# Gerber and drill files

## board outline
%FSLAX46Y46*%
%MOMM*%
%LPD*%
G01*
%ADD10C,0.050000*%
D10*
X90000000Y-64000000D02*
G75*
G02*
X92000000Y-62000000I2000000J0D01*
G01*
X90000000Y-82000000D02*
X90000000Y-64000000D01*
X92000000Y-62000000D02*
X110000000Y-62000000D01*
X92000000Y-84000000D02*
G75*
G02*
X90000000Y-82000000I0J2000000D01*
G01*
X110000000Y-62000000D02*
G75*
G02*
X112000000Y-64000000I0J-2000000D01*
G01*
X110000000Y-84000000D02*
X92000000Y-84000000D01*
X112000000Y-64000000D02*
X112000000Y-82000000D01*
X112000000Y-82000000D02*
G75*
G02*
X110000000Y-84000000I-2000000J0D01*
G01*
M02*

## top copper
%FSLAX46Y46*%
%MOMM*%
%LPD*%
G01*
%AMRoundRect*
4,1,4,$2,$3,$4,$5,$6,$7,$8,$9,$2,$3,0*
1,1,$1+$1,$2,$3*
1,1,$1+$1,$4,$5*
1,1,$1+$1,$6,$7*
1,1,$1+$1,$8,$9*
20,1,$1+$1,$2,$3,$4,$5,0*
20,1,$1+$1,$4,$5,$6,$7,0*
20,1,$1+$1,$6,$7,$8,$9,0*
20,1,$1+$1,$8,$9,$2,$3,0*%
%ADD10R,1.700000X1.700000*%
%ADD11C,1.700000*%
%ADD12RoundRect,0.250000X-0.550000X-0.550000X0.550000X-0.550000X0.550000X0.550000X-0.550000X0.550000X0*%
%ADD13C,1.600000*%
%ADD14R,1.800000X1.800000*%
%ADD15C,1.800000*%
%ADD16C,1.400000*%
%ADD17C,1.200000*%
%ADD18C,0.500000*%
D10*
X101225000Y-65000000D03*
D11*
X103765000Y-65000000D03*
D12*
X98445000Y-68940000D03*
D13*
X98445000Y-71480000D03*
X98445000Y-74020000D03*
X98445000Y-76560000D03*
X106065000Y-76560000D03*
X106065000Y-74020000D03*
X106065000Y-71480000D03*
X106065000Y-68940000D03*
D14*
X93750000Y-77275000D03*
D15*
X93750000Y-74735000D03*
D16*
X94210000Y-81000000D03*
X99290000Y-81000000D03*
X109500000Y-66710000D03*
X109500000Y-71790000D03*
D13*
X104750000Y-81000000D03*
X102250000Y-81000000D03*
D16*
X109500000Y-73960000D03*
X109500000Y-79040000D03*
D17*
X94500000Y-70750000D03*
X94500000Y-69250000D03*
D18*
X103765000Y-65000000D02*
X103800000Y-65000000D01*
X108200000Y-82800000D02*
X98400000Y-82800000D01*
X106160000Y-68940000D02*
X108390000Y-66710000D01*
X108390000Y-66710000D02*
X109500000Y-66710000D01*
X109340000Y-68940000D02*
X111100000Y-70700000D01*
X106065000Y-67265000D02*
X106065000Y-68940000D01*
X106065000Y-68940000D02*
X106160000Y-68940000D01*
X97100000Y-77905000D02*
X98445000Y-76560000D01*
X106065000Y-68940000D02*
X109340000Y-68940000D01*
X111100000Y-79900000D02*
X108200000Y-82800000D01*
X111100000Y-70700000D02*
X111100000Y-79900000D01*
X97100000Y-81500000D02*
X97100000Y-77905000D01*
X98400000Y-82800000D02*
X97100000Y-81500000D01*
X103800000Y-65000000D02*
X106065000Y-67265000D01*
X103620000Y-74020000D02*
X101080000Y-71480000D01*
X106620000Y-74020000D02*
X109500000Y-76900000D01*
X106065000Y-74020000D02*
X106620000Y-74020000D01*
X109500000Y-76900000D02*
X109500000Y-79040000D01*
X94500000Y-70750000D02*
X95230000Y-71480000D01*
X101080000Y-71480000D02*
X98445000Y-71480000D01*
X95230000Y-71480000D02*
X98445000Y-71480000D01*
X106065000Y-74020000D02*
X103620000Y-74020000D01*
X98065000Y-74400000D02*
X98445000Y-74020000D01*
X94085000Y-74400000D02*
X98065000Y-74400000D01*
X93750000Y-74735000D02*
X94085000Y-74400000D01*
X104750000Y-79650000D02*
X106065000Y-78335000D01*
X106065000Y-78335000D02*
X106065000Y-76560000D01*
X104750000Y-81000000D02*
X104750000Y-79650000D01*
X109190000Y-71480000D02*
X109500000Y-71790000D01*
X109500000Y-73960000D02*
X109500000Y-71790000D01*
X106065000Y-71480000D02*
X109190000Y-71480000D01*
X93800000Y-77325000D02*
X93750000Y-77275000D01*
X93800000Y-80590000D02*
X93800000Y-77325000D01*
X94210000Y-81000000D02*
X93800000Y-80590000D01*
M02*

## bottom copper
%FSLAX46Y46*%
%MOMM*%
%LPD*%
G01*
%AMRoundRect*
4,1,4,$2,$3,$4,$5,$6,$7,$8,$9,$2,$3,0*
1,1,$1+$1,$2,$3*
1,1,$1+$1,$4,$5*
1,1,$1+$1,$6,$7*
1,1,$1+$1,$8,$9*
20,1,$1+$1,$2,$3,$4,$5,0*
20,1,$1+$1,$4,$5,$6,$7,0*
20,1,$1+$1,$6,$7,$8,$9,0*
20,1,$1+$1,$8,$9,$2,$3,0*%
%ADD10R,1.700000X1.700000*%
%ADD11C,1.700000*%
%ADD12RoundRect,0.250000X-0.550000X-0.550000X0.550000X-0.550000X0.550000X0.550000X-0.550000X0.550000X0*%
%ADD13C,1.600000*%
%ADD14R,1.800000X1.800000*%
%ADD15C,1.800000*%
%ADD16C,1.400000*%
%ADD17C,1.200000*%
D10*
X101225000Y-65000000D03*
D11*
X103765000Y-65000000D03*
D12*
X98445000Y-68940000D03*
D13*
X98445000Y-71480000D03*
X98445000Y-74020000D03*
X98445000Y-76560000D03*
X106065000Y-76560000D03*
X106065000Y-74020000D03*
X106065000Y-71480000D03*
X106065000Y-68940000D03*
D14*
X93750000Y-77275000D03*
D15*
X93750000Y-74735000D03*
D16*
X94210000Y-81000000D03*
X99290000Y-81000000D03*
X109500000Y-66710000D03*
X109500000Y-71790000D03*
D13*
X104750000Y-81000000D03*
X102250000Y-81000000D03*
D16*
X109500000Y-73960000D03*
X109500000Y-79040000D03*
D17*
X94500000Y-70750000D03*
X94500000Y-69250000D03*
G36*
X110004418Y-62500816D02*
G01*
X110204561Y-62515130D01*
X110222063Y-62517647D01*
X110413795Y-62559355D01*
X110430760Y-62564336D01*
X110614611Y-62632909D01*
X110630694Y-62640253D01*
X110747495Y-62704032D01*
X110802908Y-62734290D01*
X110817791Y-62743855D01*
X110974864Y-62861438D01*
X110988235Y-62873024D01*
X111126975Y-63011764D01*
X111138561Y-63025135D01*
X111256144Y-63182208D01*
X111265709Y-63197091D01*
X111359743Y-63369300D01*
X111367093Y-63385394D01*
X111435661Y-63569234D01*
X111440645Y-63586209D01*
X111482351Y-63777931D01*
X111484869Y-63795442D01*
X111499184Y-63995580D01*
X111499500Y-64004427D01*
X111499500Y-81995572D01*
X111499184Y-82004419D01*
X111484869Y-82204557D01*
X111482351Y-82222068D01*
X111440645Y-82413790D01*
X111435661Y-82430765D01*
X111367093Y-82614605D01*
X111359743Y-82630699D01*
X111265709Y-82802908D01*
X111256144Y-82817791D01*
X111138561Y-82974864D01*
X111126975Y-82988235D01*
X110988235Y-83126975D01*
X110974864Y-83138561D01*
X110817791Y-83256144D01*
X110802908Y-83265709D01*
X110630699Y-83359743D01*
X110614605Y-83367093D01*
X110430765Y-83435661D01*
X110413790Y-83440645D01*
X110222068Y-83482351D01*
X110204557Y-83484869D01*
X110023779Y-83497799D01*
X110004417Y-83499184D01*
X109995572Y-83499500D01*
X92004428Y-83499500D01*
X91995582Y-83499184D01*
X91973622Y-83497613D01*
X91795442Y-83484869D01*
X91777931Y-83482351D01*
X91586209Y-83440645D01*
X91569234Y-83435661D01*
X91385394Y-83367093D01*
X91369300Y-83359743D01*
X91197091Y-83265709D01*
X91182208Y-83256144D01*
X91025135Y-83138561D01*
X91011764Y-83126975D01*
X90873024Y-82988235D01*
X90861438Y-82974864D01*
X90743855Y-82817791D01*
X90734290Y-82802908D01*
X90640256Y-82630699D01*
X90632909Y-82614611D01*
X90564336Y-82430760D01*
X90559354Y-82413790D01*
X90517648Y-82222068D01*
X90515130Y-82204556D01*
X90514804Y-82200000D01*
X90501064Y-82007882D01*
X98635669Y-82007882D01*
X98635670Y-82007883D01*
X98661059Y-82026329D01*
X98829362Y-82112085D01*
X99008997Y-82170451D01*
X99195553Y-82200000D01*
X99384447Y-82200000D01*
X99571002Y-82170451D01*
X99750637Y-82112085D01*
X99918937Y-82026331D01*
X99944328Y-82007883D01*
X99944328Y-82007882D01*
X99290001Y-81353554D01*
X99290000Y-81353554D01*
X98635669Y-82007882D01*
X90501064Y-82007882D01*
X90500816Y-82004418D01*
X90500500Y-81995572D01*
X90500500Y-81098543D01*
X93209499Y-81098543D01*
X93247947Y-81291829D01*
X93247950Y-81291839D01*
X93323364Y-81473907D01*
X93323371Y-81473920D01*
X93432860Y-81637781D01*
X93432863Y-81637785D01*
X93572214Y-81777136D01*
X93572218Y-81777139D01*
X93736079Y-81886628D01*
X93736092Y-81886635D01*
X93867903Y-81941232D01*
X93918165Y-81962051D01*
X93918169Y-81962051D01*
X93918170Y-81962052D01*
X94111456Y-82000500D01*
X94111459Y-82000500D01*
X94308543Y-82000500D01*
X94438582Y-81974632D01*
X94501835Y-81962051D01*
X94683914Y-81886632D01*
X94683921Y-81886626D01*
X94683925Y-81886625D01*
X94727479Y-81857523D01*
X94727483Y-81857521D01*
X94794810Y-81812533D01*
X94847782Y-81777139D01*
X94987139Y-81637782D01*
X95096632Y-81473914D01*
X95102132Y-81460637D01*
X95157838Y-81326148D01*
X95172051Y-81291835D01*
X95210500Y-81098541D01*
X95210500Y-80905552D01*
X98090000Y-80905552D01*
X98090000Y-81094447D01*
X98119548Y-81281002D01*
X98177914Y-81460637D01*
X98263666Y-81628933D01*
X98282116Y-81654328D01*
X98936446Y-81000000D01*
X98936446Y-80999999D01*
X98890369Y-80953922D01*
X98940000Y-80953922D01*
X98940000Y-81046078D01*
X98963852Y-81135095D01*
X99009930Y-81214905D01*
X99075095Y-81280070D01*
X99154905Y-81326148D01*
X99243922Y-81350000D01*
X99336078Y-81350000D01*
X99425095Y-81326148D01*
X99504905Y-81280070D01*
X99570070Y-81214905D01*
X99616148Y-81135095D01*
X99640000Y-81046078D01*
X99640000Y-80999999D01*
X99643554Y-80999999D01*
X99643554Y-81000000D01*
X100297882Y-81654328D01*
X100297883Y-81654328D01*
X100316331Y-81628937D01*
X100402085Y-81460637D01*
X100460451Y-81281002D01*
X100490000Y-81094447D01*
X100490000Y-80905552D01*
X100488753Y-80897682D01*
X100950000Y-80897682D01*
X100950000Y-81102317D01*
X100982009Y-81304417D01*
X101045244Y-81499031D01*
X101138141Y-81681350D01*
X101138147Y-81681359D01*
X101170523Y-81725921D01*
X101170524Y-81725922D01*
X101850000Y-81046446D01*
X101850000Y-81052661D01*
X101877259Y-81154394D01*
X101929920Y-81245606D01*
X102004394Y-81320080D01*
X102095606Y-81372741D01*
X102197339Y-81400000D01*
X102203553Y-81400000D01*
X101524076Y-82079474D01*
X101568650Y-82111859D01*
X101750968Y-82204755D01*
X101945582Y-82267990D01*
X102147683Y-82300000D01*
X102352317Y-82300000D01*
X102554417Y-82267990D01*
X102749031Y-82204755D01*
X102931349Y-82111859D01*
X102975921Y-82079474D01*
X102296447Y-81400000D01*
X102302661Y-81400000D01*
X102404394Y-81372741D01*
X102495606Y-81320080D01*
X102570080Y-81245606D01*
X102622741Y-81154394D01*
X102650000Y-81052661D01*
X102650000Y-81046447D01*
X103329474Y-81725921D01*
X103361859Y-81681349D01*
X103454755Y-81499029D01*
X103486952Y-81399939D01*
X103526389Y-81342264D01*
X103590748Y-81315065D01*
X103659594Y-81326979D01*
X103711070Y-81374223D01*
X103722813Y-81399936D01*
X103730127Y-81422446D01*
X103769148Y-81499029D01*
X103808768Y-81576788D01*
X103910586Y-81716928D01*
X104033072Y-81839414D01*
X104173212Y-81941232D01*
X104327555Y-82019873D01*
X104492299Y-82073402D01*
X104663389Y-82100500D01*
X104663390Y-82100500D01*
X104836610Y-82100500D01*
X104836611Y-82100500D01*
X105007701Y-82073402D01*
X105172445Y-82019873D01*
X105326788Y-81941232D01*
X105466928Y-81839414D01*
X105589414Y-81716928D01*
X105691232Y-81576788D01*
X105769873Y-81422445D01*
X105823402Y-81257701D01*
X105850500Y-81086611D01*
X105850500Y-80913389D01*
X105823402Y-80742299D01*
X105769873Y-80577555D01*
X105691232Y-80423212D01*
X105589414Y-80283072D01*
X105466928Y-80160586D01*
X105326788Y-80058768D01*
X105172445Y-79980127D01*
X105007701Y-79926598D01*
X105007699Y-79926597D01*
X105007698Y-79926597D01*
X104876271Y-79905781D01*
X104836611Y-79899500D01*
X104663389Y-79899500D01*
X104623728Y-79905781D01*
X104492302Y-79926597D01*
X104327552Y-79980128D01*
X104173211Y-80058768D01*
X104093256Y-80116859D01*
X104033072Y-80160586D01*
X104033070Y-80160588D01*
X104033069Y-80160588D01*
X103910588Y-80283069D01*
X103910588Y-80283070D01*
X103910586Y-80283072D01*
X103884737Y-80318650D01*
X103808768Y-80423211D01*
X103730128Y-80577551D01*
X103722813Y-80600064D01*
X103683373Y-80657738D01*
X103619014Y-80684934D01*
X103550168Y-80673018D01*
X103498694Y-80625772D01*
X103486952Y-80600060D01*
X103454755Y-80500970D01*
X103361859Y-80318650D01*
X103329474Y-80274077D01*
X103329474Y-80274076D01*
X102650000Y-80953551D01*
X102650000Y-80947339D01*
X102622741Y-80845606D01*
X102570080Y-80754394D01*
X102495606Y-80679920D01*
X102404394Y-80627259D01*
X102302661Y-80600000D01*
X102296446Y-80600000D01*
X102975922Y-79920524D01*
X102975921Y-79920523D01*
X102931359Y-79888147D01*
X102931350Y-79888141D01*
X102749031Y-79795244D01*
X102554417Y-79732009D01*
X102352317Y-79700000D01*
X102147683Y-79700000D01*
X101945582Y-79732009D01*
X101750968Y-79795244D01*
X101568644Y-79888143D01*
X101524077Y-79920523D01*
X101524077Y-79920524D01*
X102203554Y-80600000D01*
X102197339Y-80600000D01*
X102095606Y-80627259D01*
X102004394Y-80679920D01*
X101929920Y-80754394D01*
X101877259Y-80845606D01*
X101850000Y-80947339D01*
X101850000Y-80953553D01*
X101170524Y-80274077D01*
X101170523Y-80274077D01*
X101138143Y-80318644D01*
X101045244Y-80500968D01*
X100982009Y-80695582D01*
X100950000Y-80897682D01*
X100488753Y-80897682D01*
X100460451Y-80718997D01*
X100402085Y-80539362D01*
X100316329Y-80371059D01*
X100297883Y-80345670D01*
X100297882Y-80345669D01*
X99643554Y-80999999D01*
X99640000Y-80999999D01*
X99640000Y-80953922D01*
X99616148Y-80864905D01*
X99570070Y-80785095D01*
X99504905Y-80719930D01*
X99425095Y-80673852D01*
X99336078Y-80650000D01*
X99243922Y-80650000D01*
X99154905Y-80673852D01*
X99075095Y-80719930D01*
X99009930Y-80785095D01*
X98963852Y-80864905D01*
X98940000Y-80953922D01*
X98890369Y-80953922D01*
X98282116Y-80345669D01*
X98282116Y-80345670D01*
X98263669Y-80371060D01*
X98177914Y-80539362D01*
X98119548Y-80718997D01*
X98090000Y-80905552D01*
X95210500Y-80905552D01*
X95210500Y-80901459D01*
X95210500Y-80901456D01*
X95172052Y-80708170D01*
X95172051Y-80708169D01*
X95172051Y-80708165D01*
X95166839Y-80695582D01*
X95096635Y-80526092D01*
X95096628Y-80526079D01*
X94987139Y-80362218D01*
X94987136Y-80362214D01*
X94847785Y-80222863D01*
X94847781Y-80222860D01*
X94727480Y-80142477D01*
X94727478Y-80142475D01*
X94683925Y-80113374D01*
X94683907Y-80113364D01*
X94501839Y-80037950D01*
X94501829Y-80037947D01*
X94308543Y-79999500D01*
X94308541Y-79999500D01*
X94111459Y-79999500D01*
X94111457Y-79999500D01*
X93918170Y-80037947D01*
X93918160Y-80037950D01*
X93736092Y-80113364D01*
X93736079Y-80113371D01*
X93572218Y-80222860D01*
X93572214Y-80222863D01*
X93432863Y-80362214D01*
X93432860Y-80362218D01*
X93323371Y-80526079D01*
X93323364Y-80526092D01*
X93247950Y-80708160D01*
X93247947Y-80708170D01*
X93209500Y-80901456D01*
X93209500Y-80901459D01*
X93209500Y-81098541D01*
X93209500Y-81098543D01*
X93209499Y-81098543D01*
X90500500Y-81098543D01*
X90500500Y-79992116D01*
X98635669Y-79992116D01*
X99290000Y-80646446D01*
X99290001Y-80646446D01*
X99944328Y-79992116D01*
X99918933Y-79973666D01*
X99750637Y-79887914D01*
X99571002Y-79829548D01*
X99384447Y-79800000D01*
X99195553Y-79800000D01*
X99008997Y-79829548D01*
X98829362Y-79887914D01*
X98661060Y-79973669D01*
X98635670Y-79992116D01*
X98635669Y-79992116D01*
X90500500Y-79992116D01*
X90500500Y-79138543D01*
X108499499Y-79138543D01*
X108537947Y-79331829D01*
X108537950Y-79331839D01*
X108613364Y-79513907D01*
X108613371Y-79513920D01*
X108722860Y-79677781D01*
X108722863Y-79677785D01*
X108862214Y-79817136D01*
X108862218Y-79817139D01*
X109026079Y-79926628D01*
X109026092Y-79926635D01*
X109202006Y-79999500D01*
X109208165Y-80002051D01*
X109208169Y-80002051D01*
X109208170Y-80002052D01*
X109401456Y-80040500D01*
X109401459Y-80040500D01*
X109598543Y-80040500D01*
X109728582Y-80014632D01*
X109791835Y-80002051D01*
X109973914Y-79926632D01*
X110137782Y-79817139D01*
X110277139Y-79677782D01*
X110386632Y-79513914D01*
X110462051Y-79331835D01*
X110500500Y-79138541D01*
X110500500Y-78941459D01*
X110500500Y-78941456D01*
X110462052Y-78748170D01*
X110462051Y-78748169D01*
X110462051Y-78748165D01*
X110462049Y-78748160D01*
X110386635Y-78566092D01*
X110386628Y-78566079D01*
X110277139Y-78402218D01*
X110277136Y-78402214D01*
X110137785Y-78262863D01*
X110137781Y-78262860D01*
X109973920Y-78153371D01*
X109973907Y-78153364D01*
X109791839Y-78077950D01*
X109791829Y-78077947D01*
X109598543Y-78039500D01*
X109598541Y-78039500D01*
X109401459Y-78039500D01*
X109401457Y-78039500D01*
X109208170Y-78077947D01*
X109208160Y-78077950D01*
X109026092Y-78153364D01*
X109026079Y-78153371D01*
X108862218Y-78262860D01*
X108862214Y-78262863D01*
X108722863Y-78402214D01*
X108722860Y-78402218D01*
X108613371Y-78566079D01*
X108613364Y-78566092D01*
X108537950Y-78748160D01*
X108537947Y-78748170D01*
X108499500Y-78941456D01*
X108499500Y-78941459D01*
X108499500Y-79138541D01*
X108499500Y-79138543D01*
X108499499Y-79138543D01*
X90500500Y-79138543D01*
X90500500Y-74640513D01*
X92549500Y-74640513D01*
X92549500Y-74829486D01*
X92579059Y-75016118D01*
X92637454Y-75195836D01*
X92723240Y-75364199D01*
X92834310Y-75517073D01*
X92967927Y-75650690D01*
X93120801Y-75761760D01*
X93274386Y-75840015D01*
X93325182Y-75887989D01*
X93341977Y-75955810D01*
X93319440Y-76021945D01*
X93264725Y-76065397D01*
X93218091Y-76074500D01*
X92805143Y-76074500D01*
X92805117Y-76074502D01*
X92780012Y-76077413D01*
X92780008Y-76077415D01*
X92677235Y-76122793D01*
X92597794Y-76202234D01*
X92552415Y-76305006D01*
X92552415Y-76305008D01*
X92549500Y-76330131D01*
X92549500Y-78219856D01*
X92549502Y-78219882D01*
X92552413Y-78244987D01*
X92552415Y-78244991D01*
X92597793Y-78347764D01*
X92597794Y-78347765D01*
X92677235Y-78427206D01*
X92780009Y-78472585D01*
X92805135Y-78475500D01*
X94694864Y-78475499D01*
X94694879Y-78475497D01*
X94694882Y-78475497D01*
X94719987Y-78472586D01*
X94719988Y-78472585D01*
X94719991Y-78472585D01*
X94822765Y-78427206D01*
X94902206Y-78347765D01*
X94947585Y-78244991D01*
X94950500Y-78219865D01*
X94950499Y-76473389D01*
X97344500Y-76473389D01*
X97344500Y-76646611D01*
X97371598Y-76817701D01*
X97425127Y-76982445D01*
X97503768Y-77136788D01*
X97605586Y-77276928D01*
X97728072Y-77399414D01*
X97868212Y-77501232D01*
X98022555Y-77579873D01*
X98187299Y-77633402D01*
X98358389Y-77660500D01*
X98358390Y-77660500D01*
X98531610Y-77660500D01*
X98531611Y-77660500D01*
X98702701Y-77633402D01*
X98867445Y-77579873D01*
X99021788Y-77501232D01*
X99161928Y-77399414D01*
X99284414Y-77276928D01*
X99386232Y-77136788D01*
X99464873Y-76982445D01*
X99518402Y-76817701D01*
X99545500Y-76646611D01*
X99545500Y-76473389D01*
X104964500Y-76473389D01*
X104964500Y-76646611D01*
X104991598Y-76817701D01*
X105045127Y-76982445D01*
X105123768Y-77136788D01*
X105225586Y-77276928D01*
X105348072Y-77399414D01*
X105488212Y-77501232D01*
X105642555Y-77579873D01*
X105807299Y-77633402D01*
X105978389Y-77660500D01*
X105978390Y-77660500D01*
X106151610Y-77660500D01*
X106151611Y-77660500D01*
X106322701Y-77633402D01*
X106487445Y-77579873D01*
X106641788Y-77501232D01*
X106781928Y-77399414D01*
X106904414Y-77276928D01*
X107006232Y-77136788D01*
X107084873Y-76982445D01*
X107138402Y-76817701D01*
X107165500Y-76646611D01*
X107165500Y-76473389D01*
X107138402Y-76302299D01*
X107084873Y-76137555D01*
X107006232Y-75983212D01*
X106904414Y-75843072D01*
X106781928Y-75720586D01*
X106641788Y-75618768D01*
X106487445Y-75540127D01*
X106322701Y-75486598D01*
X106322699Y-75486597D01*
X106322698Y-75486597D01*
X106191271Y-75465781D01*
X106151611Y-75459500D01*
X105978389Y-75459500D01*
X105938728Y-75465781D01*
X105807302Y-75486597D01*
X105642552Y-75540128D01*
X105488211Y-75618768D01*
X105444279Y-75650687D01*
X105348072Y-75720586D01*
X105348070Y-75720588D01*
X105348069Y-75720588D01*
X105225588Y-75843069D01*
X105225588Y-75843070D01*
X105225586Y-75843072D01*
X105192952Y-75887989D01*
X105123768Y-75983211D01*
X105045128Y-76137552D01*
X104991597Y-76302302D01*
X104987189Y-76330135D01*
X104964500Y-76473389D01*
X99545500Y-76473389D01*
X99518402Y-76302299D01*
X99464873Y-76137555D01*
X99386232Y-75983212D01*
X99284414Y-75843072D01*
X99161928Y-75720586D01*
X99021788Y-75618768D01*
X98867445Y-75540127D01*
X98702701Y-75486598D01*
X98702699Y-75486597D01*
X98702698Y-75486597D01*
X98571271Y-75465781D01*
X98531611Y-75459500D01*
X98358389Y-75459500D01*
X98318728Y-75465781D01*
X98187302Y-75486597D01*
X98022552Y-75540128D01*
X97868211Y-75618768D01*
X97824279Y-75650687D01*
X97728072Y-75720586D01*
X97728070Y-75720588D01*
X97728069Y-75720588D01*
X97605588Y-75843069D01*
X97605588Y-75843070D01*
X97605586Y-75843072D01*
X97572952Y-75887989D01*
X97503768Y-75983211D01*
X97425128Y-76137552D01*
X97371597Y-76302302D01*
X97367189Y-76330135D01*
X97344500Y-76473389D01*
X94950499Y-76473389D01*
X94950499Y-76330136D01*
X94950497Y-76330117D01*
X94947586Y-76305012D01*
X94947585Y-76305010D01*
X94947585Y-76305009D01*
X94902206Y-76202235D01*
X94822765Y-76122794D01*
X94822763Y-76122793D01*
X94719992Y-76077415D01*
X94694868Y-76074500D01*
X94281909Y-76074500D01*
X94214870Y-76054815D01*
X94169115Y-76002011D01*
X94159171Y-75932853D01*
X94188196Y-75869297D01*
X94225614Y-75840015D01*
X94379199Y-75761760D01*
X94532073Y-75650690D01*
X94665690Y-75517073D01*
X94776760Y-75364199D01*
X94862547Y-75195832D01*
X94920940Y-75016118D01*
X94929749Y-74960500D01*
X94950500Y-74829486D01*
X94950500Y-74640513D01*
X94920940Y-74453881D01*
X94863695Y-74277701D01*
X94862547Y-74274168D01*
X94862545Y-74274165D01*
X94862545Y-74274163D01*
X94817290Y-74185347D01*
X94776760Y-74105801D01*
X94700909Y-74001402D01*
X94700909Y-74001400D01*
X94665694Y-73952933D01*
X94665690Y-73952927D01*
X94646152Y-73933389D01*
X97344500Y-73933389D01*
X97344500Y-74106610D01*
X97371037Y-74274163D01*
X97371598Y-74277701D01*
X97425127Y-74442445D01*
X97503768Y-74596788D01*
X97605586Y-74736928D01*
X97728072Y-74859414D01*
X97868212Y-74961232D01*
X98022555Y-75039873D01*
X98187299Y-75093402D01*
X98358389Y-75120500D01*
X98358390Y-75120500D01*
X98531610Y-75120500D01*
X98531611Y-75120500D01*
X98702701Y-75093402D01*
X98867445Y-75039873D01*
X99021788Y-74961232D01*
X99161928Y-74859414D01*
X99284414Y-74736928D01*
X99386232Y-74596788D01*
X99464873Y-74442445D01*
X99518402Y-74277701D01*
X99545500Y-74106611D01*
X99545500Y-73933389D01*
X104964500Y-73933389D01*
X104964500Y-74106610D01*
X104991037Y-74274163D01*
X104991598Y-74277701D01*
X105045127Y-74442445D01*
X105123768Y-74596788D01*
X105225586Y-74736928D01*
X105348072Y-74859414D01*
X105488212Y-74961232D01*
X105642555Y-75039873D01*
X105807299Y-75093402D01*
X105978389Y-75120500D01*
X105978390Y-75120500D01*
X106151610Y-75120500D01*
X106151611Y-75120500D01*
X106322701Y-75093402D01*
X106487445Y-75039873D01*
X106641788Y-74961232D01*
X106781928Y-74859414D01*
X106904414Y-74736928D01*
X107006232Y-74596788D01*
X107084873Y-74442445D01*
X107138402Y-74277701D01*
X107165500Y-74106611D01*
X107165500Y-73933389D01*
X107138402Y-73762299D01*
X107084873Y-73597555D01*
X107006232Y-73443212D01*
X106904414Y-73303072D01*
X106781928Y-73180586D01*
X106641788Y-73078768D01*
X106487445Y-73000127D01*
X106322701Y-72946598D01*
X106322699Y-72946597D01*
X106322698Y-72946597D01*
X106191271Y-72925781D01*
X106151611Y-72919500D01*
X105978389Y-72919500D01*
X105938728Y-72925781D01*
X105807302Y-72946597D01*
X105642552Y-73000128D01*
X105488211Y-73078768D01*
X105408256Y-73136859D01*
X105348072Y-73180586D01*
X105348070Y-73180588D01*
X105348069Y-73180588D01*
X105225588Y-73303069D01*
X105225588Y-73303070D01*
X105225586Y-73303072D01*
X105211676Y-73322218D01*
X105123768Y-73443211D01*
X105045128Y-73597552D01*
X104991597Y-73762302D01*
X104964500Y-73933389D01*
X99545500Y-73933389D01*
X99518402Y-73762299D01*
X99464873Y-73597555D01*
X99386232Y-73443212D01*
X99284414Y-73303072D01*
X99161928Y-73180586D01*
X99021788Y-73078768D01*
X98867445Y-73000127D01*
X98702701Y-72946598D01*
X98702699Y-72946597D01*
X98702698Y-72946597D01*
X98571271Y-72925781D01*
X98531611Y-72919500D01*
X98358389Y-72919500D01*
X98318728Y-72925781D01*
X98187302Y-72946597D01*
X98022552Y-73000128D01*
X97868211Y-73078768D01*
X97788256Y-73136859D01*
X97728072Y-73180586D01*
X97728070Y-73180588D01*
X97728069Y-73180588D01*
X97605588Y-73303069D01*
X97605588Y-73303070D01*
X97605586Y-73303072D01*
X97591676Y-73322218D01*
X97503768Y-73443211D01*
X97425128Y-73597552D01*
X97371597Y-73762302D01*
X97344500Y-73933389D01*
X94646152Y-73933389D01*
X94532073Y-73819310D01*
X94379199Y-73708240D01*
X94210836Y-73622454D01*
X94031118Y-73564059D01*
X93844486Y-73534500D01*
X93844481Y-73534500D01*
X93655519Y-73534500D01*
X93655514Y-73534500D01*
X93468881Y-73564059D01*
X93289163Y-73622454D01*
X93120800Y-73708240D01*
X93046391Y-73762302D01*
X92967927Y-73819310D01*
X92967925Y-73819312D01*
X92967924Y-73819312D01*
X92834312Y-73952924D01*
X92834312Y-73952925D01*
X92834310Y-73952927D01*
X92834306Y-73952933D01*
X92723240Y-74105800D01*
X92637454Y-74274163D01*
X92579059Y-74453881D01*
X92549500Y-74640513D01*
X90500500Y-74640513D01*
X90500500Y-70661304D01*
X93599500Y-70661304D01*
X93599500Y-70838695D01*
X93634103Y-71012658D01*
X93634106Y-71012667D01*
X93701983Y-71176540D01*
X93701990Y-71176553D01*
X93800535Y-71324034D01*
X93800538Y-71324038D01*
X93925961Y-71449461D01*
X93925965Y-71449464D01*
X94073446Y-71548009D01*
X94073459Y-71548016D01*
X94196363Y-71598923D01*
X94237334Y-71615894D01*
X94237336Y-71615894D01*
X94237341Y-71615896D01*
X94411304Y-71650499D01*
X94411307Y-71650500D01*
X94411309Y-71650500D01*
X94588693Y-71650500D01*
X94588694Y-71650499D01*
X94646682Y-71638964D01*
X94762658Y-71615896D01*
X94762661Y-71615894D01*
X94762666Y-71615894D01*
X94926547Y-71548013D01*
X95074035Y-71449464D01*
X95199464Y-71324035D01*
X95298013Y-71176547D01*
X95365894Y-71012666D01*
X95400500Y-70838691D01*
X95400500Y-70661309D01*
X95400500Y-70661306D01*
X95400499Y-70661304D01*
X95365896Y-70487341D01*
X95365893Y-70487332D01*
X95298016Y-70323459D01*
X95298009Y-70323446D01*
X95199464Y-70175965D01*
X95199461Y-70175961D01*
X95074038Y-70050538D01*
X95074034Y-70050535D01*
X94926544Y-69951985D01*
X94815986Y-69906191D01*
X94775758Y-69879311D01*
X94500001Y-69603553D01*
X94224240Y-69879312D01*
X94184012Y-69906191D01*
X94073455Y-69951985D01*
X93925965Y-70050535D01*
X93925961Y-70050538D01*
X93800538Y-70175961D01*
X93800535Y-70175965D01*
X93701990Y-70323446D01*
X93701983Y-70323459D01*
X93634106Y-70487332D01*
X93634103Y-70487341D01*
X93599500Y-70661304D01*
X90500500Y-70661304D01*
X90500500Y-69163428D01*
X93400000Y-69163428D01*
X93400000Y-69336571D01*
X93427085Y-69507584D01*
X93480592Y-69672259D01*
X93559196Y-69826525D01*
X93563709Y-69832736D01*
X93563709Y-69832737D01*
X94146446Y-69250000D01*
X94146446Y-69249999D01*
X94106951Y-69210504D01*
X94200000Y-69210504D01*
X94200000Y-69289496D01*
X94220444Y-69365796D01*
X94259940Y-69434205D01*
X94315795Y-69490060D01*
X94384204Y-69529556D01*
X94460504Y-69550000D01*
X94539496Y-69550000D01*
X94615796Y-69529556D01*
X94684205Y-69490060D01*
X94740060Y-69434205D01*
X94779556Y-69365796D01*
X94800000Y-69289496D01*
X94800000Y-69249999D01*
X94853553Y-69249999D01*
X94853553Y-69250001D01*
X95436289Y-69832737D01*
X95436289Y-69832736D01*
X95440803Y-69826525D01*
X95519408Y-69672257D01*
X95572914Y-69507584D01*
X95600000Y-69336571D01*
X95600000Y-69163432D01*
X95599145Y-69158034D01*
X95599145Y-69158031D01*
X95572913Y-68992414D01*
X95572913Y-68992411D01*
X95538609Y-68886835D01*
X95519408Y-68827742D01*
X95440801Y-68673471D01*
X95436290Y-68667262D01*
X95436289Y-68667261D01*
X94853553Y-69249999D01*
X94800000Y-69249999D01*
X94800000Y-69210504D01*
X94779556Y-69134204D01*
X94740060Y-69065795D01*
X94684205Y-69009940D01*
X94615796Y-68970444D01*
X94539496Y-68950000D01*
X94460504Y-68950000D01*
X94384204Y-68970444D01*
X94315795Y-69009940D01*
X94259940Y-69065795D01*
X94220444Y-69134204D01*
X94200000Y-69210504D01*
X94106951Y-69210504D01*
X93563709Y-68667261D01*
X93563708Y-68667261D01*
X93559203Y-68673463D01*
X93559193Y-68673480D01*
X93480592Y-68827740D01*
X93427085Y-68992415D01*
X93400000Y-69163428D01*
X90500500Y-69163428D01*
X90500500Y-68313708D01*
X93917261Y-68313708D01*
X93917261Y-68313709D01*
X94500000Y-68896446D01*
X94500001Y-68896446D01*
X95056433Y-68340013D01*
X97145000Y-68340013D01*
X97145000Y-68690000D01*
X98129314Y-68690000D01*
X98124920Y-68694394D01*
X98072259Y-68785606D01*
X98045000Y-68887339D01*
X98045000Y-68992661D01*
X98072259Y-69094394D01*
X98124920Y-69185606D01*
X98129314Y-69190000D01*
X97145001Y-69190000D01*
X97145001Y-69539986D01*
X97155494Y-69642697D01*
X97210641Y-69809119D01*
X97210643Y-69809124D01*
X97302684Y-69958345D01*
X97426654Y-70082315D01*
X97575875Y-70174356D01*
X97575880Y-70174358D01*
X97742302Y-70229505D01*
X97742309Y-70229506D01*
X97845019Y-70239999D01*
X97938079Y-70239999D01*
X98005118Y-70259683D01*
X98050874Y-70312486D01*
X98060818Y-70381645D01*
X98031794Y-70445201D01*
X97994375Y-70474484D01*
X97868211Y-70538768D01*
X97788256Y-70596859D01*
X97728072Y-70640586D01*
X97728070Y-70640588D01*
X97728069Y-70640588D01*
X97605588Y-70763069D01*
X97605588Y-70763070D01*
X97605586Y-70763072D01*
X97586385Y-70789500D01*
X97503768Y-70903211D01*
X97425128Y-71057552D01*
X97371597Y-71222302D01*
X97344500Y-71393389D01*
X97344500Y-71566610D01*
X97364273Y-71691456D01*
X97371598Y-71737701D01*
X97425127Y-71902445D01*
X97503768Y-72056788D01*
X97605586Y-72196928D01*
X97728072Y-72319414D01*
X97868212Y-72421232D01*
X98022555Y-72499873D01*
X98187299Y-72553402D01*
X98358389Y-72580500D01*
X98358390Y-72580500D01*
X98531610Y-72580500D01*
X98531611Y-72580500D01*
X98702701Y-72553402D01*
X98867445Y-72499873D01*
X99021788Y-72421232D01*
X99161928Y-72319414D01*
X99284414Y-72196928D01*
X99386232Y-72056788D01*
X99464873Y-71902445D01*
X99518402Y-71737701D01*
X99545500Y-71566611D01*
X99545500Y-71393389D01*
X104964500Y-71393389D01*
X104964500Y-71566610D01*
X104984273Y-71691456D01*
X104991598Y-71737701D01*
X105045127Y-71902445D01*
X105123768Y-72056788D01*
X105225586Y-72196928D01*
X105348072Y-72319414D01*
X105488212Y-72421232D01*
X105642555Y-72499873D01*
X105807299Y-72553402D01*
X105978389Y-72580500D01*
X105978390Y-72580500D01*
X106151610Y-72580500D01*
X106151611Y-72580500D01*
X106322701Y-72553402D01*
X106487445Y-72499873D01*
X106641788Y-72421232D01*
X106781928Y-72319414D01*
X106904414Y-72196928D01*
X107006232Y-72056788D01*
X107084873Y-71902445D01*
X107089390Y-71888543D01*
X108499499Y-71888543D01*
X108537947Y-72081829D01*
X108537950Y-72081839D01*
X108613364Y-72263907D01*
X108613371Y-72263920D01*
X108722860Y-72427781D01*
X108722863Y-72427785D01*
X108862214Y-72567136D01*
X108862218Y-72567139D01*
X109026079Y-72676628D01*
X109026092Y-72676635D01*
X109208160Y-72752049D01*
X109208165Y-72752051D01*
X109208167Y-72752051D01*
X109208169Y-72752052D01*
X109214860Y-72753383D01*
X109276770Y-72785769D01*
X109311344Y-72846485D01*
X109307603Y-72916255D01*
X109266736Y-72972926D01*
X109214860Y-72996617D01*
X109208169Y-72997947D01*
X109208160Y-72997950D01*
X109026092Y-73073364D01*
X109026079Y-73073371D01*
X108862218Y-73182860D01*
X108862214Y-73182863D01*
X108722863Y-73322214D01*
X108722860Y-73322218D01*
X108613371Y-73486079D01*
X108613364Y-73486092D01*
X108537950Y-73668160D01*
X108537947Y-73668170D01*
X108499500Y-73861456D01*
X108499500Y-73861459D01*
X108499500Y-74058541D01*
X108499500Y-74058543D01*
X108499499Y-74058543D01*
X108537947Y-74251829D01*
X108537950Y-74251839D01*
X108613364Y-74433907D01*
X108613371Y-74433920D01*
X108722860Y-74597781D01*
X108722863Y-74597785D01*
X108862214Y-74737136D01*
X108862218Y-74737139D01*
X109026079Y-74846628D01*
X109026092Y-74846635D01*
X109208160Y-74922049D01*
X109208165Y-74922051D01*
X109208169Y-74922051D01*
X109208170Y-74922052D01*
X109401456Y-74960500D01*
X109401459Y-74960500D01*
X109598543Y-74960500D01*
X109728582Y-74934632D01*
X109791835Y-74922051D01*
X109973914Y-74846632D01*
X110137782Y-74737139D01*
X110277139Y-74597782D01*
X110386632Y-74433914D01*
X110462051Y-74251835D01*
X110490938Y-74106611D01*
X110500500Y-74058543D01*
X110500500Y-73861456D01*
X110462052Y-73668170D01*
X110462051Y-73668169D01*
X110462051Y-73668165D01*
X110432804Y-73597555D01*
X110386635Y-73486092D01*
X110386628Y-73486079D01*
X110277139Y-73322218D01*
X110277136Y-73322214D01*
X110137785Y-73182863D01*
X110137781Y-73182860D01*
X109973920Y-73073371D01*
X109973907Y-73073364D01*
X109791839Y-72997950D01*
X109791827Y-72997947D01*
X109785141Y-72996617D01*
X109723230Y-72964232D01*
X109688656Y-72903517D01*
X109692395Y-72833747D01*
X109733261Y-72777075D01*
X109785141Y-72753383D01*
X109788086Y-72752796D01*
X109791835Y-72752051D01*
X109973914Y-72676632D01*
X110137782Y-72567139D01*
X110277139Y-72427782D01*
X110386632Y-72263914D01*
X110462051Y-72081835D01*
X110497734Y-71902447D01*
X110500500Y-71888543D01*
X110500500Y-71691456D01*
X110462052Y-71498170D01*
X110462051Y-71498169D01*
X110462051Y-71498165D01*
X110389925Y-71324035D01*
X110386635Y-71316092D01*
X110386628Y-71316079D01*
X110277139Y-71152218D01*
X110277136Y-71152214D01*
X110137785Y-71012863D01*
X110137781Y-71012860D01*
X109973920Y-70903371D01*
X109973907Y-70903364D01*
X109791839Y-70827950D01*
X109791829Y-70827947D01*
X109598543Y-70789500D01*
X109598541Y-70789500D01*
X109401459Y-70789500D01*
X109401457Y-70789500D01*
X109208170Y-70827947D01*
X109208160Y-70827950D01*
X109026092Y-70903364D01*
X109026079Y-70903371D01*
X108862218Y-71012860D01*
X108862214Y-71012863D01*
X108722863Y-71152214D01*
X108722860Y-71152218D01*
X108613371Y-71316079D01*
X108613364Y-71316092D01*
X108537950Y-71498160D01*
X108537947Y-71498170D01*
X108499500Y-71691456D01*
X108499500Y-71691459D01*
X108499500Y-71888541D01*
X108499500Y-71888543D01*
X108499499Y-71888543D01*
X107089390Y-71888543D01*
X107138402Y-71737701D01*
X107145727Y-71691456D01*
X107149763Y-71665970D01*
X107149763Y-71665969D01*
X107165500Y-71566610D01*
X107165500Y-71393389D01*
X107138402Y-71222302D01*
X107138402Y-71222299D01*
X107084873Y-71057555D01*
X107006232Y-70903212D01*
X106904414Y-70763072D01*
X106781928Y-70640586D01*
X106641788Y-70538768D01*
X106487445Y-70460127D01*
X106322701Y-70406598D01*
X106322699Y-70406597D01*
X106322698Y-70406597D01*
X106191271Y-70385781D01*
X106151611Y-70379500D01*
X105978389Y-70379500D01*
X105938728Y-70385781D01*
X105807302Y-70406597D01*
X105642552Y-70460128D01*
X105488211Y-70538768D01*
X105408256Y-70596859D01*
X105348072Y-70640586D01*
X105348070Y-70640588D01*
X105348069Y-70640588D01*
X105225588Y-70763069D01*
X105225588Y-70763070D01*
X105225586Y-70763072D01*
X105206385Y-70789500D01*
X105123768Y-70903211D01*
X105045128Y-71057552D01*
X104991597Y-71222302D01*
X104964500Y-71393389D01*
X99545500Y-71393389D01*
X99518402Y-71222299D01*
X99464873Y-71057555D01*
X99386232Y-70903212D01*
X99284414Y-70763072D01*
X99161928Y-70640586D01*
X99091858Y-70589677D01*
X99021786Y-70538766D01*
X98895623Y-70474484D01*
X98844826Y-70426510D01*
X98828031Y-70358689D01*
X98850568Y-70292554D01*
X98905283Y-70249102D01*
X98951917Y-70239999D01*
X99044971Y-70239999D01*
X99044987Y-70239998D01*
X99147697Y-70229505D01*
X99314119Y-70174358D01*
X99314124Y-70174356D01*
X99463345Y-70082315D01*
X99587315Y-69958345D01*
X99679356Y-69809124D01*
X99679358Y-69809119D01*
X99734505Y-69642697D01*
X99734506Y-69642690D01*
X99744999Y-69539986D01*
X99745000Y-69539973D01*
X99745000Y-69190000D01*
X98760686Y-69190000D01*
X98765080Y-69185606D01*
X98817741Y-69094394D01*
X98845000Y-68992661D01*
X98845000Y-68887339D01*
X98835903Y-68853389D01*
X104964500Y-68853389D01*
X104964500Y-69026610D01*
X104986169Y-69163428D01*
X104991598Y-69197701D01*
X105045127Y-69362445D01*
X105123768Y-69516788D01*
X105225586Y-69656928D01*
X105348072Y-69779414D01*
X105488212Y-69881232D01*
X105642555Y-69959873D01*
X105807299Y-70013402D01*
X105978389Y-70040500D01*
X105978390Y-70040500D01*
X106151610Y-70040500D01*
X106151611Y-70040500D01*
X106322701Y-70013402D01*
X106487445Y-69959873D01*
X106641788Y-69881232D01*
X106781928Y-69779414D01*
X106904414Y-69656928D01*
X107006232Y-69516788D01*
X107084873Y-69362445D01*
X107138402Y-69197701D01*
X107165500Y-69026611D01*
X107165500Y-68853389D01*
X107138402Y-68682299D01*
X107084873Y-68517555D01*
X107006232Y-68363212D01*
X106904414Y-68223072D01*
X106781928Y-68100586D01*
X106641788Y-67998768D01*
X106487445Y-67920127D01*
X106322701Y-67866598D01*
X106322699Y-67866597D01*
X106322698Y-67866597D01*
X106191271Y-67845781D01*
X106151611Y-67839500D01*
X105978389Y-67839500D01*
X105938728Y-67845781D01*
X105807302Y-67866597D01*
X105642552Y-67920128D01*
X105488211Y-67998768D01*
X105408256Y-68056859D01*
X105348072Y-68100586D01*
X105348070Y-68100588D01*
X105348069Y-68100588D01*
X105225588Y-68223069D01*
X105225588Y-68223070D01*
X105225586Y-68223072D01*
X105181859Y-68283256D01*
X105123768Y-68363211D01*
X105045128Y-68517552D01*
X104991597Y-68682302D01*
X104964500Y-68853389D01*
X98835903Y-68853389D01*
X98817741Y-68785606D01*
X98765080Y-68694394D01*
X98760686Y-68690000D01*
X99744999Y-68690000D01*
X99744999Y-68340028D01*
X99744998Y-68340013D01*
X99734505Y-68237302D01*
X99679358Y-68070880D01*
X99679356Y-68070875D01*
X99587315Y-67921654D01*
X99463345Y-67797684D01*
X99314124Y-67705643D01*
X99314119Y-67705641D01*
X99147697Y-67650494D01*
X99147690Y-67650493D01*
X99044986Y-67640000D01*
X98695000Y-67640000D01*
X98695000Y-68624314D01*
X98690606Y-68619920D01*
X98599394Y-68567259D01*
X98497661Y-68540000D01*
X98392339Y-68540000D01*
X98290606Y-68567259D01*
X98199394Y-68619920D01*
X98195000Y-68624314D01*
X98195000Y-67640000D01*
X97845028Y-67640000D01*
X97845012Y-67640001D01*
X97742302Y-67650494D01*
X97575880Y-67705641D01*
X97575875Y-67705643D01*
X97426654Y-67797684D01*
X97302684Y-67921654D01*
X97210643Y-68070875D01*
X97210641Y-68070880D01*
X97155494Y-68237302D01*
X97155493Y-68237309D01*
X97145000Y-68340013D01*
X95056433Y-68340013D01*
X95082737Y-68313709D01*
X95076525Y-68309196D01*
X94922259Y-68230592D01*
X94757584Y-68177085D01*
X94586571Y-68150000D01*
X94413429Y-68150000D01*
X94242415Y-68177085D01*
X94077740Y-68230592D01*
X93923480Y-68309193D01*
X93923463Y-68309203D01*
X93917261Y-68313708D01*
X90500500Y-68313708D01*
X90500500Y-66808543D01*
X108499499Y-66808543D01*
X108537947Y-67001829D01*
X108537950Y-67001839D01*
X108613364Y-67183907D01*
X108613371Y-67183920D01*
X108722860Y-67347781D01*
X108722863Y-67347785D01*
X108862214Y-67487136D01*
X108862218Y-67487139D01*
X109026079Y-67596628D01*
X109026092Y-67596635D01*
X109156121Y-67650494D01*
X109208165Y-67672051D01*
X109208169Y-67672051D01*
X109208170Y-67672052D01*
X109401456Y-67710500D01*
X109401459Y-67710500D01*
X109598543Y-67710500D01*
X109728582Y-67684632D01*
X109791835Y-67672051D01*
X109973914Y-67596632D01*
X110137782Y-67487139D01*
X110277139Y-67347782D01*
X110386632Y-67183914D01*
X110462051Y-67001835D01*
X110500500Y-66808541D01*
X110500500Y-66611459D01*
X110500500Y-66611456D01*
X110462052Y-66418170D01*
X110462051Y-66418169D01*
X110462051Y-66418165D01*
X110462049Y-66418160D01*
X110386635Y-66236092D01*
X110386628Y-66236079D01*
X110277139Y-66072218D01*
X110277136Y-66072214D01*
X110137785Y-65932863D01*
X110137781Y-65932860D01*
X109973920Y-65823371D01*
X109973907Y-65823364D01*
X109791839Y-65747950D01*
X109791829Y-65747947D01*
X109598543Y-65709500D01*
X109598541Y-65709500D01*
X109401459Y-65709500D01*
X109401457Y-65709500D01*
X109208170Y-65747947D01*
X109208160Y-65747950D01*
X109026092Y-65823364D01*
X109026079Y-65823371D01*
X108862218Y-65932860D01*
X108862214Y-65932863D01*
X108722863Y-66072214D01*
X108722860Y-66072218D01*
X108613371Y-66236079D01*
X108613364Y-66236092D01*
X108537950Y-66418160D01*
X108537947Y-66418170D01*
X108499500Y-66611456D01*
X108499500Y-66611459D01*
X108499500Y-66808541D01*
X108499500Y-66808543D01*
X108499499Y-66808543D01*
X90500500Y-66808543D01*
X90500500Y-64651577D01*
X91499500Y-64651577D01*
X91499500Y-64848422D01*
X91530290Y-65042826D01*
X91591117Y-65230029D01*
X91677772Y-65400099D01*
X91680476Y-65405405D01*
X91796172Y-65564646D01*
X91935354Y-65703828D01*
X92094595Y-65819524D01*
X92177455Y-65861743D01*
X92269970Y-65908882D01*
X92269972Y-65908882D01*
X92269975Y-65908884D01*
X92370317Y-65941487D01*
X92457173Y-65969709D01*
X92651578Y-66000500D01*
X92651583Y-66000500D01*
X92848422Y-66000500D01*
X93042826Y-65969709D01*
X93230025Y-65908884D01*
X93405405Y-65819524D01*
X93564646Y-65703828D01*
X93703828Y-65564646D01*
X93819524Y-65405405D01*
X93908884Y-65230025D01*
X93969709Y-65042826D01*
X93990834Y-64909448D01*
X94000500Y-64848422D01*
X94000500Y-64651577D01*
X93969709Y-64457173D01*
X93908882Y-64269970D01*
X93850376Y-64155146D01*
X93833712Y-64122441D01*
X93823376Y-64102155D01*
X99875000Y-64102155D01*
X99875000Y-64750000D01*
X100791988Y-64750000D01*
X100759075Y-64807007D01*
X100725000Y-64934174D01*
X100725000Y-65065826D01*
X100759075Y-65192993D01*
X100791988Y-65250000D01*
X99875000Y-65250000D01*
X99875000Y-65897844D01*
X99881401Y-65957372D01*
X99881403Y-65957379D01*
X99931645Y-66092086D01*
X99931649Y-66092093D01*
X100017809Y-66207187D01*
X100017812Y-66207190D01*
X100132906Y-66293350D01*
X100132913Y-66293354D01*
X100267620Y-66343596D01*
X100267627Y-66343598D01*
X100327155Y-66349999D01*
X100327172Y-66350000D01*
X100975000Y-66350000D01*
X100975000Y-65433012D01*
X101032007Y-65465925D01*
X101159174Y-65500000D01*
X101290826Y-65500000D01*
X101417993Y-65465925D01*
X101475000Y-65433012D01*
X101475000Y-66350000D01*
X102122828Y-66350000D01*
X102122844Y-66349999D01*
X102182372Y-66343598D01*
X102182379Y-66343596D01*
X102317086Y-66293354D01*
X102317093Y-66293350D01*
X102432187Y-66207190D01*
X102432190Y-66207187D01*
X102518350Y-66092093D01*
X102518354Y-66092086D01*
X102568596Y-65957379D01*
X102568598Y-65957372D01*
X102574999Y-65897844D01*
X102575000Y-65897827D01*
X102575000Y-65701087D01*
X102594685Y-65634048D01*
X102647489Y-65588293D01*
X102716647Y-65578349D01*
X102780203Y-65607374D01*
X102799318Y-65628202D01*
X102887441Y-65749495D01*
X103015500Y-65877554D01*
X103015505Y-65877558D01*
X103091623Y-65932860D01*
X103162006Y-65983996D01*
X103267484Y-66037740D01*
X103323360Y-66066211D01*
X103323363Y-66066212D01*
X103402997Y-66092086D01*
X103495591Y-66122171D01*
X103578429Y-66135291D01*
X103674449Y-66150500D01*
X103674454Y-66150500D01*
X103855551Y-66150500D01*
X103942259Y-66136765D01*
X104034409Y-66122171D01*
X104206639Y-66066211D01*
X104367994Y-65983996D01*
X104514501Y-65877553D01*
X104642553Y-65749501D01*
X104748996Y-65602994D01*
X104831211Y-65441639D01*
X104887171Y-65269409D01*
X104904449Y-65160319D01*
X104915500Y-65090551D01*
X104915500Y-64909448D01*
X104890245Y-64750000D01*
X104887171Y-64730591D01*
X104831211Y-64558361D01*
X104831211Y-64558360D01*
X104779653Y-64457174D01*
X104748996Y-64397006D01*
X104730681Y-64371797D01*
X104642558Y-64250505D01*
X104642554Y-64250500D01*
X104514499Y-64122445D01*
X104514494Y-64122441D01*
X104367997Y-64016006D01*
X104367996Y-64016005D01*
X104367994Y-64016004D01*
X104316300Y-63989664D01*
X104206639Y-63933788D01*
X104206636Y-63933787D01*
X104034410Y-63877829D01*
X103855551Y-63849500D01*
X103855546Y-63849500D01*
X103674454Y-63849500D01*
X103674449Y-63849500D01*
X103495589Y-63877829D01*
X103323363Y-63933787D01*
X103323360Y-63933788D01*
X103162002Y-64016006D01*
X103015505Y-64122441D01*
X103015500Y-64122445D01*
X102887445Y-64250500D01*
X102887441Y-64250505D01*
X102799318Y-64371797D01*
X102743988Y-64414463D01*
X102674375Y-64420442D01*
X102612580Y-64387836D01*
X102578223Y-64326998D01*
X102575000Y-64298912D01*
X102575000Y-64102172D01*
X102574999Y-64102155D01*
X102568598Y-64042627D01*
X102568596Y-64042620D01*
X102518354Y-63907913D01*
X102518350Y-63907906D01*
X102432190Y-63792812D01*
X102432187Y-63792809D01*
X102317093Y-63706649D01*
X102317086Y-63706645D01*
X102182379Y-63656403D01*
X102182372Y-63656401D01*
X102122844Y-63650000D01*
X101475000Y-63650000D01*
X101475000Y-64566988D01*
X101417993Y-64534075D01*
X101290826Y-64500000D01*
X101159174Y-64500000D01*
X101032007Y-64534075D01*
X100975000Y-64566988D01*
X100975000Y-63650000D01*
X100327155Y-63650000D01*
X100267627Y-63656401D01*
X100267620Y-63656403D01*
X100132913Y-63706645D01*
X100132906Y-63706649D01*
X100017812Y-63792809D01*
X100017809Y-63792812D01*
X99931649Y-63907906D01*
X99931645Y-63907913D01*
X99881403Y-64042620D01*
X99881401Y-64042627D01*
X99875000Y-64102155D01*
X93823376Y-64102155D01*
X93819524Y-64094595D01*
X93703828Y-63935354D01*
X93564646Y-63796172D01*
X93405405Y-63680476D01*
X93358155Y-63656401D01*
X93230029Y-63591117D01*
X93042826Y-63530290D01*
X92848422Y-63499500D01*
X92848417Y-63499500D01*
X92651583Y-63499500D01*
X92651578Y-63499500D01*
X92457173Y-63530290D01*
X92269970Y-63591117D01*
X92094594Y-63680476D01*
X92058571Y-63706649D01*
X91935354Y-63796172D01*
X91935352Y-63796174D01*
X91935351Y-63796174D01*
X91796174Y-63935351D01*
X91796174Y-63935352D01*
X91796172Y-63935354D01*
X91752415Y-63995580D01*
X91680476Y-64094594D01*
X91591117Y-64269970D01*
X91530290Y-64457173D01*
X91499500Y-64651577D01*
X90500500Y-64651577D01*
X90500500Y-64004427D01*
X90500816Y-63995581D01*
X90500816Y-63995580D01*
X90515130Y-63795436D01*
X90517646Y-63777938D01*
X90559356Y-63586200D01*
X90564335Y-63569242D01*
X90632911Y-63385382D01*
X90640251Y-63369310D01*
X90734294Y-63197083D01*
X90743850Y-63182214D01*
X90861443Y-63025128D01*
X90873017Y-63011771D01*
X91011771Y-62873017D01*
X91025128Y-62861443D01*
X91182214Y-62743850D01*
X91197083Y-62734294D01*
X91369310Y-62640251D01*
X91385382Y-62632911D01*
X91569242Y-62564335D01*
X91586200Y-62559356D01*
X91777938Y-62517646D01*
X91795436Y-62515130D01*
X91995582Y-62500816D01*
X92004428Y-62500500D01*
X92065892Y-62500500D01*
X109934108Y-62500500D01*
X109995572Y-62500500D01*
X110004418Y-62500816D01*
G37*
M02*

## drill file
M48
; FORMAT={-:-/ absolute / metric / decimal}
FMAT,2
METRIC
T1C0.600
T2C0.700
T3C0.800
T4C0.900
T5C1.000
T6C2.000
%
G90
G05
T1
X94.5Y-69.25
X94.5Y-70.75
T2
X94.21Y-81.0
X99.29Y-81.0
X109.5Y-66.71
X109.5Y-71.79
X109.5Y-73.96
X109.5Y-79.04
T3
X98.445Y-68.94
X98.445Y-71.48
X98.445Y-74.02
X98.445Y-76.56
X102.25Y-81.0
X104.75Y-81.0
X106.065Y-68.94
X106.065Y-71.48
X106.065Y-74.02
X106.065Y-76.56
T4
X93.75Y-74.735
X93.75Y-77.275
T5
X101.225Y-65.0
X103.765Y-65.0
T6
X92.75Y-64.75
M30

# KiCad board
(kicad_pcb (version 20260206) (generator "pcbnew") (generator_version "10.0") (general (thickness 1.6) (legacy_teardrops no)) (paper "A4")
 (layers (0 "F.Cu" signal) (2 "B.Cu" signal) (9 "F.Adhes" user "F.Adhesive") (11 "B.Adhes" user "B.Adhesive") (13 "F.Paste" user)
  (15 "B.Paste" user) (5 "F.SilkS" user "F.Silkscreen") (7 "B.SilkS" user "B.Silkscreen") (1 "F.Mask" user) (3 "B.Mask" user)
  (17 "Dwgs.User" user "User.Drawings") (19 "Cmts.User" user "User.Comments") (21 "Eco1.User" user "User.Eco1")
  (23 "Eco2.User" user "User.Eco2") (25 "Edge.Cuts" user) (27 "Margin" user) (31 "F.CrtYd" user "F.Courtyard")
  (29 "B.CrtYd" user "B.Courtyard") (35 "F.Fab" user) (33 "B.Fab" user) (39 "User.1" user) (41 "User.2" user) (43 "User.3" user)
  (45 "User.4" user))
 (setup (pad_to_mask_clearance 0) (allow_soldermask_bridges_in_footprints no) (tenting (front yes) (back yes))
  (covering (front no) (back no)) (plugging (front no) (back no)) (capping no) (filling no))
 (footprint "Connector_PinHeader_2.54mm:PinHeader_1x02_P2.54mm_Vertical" (layer "F.Cu") (at 101.225 65 90)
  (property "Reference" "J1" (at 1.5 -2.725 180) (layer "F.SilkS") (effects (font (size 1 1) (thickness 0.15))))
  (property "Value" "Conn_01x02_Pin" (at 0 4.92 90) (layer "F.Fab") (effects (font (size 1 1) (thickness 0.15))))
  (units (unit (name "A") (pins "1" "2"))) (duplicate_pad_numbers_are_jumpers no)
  (pad "1" thru_hole rect (at 0 0 90) (size 1.7 1.7) (drill 1) (layers "*.Cu" "*.Mask") (remove_unused_layers no) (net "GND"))
  (pad "2" thru_hole circle (at 0 2.54 90) (size 1.7 1.7) (drill 1) (layers "*.Cu" "*.Mask") (remove_unused_layers no) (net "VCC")))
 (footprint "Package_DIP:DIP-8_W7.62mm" (layer "F.Cu") (at 98.445 68.94)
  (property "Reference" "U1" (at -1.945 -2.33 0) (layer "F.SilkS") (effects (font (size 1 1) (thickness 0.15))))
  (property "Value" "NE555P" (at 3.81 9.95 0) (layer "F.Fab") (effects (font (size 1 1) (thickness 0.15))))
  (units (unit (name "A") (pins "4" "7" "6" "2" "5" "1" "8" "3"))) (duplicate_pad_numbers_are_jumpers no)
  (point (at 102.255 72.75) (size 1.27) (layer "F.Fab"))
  (pad "1" thru_hole roundrect (at 0 0) (size 1.6 1.6) (drill 0.8) (layers "*.Cu" "*.Mask") (remove_unused_layers no)
   (roundrect_rratio 0.15625) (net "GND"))
  (pad "2" thru_hole circle (at 0 2.54) (size 1.6 1.6) (drill 0.8) (layers "*.Cu" "*.Mask") (remove_unused_layers no) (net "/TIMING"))
  (pad "3" thru_hole circle (at 0 5.08) (size 1.6 1.6) (drill 0.8) (layers "*.Cu" "*.Mask") (remove_unused_layers no) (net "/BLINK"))
  (pad "4" thru_hole circle (at 0 7.62) (size 1.6 1.6) (drill 0.8) (layers "*.Cu" "*.Mask") (remove_unused_layers no) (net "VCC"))
  (pad "5" thru_hole circle (at 7.62 7.62) (size 1.6 1.6) (drill 0.8) (layers "*.Cu" "*.Mask") (remove_unused_layers no)
   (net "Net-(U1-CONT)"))
  (pad "6" thru_hole circle (at 7.62 5.08) (size 1.6 1.6) (drill 0.8) (layers "*.Cu" "*.Mask") (remove_unused_layers no) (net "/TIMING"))
  (pad "7" thru_hole circle (at 7.62 2.54) (size 1.6 1.6) (drill 0.8) (layers "*.Cu" "*.Mask") (remove_unused_layers no) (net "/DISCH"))
  (pad "8" thru_hole circle (at 7.62 0) (size 1.6 1.6) (drill 0.8) (layers "*.Cu" "*.Mask") (remove_unused_layers no) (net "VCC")))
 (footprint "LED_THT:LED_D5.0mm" (layer "F.Cu") (at 93.75 77.275 90)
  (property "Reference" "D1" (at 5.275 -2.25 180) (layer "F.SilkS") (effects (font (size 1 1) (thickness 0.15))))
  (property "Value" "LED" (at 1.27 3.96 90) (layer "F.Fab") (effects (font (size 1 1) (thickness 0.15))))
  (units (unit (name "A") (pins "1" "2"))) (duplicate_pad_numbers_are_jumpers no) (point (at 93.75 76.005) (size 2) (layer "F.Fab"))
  (pad "1" thru_hole rect (at 0 0 90) (size 1.8 1.8) (drill 0.9) (layers "*.Cu" "*.Mask") (remove_unused_layers no) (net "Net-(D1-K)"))
  (pad "2" thru_hole circle (at 2.54 0 90) (size 1.8 1.8) (drill 0.9) (layers "*.Cu" "*.Mask") (remove_unused_layers no) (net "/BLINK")))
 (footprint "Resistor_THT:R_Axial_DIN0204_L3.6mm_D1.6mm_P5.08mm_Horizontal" (layer "F.Cu") (at 94.21 81)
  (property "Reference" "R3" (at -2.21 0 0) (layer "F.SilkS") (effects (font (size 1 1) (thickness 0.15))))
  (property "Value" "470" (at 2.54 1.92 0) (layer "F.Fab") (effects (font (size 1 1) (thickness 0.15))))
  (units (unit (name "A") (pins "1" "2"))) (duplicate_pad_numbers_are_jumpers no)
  (pad "1" thru_hole circle (at 0 0) (size 1.4 1.4) (drill 0.7) (layers "*.Cu" "*.Mask") (remove_unused_layers no) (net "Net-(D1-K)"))
  (pad "2" thru_hole circle (at 5.08 0) (size 1.4 1.4) (drill 0.7) (layers "*.Cu" "*.Mask") (remove_unused_layers no) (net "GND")))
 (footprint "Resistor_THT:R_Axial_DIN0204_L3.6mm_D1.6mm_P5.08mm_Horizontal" (layer "F.Cu") (at 109.5 66.71 -90)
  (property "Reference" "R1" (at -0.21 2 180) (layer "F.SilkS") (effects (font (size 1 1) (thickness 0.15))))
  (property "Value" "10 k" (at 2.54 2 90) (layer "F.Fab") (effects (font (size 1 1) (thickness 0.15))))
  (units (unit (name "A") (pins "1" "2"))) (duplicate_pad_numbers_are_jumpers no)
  (pad "1" thru_hole circle (at 0 0 270) (size 1.4 1.4) (drill 0.7) (layers "*.Cu" "*.Mask") (remove_unused_layers no) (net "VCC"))
  (pad "2" thru_hole circle (at 5.08 0 270) (size 1.4 1.4) (drill 0.7) (layers "*.Cu" "*.Mask") (remove_unused_layers no) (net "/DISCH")))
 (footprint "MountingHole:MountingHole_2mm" (layer "F.Cu") (at 92.75 64.75)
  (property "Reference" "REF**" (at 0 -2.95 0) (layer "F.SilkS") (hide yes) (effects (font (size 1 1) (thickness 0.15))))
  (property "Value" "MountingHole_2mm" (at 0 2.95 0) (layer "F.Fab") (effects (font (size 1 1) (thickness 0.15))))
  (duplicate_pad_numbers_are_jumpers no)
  (pad "" np_thru_hole circle (at 0 0) (size 2 2) (drill 2) (layers "*.Cu" "*.Mask")))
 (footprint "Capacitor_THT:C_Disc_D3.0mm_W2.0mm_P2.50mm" (layer "F.Cu") (at 104.75 81 180)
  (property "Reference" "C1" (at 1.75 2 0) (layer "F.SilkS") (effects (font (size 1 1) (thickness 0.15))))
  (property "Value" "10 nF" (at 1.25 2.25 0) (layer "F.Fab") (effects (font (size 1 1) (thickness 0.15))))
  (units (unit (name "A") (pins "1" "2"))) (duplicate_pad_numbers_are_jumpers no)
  (pad "1" thru_hole circle (at 0 0 180) (size 1.6 1.6) (drill 0.8) (layers "*.Cu" "*.Mask") (remove_unused_layers no) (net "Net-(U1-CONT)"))
  (pad "2" thru_hole circle (at 2.5 0 180) (size 1.6 1.6) (drill 0.8) (layers "*.Cu" "*.Mask") (remove_unused_layers no) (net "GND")))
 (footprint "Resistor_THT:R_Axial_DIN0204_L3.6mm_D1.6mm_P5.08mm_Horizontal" (layer "F.Cu") (at 109.5 73.96 -90)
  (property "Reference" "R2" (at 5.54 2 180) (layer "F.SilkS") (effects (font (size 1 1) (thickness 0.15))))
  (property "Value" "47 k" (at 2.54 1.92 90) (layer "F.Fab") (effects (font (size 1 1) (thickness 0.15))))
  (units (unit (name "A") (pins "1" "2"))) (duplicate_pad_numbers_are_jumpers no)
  (pad "1" thru_hole circle (at 0 0 270) (size 1.4 1.4) (drill 0.7) (layers "*.Cu" "*.Mask") (remove_unused_layers no) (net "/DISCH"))
  (pad "2" thru_hole circle (at 5.08 0 270) (size 1.4 1.4) (drill 0.7) (layers "*.Cu" "*.Mask") (remove_unused_layers no) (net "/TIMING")))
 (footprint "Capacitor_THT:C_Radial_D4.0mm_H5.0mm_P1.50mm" (layer "F.Cu") (at 94.5 70.75 90)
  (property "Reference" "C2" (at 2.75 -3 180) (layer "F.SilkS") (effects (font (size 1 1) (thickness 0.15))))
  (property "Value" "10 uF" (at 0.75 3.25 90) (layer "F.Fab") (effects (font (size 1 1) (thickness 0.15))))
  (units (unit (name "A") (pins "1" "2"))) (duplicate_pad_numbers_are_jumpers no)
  (pad "1" thru_hole circle (at 0 0 90) (size 1.2 1.2) (drill 0.6) (layers "*.Cu" "*.Mask") (remove_unused_layers no) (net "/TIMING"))
  (pad "2" thru_hole circle (at 1.5 0 90) (size 1.2 1.2) (drill 0.6) (layers "*.Cu" "*.Mask") (remove_unused_layers no) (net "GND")))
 (gr_arc (start 90 64) (mid 90.585786 62.585786) (end 92 62) (stroke (width 0.05) (type default)) (layer "Edge.Cuts"))
 (gr_line (start 90 82) (end 90 64) (stroke (width 0.05) (type default)) (layer "Edge.Cuts"))
 (gr_line (start 92 62) (end 110 62) (stroke (width 0.05) (type default)) (layer "Edge.Cuts"))
 (gr_arc (start 92 84) (mid 90.585786 83.414214) (end 90 82) (stroke (width 0.05) (type default)) (layer "Edge.Cuts"))
 (gr_arc (start 110 62) (mid 111.414214 62.585786) (end 112 64) (stroke (width 0.05) (type default)) (layer "Edge.Cuts"))
 (gr_line (start 110 84) (end 92 84) (stroke (width 0.05) (type default)) (layer "Edge.Cuts"))
 (gr_line (start 112 64) (end 112 82) (stroke (width 0.05) (type default)) (layer "Edge.Cuts"))
 (gr_arc (start 112 82) (mid 111.414214 83.414214) (end 110 84) (stroke (width 0.05) (type default)) (layer "Edge.Cuts"))
 (segment (start 103.765 65) (end 103.8 65) (width 0.5) (layer "F.Cu") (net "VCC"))
 (segment (start 108.2 82.8) (end 98.4 82.8) (width 0.5) (layer "F.Cu") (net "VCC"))
 (segment (start 106.16 68.94) (end 108.39 66.71) (width 0.5) (layer "F.Cu") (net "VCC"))
 (segment (start 108.39 66.71) (end 109.5 66.71) (width 0.5) (layer "F.Cu") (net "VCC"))
 (segment (start 109.34 68.94) (end 111.1 70.7) (width 0.5) (layer "F.Cu") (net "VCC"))
 (segment (start 106.065 67.265) (end 106.065 68.94) (width 0.5) (layer "F.Cu") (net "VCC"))
 (segment (start 106.065 68.94) (end 106.16 68.94) (width 0.5) (layer "F.Cu") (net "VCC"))
 (segment (start 97.1 77.905) (end 98.445 76.56) (width 0.5) (layer "F.Cu") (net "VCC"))
 (segment (start 106.065 68.94) (end 109.34 68.94) (width 0.5) (layer "F.Cu") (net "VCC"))
 (segment (start 111.1 79.9) (end 108.2 82.8) (width 0.5) (layer "F.Cu") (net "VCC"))
 (segment (start 111.1 70.7) (end 111.1 79.9) (width 0.5) (layer "F.Cu") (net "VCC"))
 (segment (start 97.1 81.5) (end 97.1 77.905) (width 0.5) (layer "F.Cu") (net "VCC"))
 (segment (start 98.4 82.8) (end 97.1 81.5) (width 0.5) (layer "F.Cu") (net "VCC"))
 (segment (start 103.8 65) (end 106.065 67.265) (width 0.5) (layer "F.Cu") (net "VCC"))
 (segment (start 103.62 74.02) (end 101.08 71.48) (width 0.5) (layer "F.Cu") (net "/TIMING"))
 (segment (start 106.62 74.02) (end 109.5 76.9) (width 0.5) (layer "F.Cu") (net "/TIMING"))
 (segment (start 106.065 74.02) (end 106.62 74.02) (width 0.5) (layer "F.Cu") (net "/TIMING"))
 (segment (start 109.5 76.9) (end 109.5 79.04) (width 0.5) (layer "F.Cu") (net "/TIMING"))
 (segment (start 94.5 70.75) (end 95.23 71.48) (width 0.5) (layer "F.Cu") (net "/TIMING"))
 (segment (start 101.08 71.48) (end 98.445 71.48) (width 0.5) (layer "F.Cu") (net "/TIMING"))
 (segment (start 95.23 71.48) (end 98.445 71.48) (width 0.5) (layer "F.Cu") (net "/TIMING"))
 (segment (start 106.065 74.02) (end 103.62 74.02) (width 0.5) (layer "F.Cu") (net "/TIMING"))
 (segment (start 98.065 74.4) (end 98.445 74.02) (width 0.5) (layer "F.Cu") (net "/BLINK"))
 (segment (start 94.085 74.4) (end 98.065 74.4) (width 0.5) (layer "F.Cu") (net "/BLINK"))
 (segment (start 93.75 74.735) (end 94.085 74.4) (width 0.5) (layer "F.Cu") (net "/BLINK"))
 (segment (start 104.75 79.65) (end 106.065 78.335) (width 0.5) (layer "F.Cu") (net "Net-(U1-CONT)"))
 (segment (start 106.065 78.335) (end 106.065 76.56) (width 0.5) (layer "F.Cu") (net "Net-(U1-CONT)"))
 (segment (start 104.75 81) (end 104.75 79.65) (width 0.5) (layer "F.Cu") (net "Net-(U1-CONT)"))
 (segment (start 109.19 71.48) (end 109.5 71.79) (width 0.5) (layer "F.Cu") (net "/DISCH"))
 (segment (start 109.5 73.96) (end 109.5 71.79) (width 0.5) (layer "F.Cu") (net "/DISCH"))
 (segment (start 106.065 71.48) (end 109.19 71.48) (width 0.5) (layer "F.Cu") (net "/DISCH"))
 (segment (start 93.8 77.325) (end 93.75 77.275) (width 0.5) (layer "F.Cu") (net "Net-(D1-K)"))
 (segment (start 93.8 80.59) (end 93.8 77.325) (width 0.5) (layer "F.Cu") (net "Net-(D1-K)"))
 (segment (start 94.21 81) (end 93.8 80.59) (width 0.5) (layer "F.Cu") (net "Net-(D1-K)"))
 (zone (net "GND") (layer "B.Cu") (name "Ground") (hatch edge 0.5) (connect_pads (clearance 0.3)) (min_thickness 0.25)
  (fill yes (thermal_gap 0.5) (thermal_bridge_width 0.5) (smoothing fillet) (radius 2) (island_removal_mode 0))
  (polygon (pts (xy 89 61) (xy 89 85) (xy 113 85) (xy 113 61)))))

